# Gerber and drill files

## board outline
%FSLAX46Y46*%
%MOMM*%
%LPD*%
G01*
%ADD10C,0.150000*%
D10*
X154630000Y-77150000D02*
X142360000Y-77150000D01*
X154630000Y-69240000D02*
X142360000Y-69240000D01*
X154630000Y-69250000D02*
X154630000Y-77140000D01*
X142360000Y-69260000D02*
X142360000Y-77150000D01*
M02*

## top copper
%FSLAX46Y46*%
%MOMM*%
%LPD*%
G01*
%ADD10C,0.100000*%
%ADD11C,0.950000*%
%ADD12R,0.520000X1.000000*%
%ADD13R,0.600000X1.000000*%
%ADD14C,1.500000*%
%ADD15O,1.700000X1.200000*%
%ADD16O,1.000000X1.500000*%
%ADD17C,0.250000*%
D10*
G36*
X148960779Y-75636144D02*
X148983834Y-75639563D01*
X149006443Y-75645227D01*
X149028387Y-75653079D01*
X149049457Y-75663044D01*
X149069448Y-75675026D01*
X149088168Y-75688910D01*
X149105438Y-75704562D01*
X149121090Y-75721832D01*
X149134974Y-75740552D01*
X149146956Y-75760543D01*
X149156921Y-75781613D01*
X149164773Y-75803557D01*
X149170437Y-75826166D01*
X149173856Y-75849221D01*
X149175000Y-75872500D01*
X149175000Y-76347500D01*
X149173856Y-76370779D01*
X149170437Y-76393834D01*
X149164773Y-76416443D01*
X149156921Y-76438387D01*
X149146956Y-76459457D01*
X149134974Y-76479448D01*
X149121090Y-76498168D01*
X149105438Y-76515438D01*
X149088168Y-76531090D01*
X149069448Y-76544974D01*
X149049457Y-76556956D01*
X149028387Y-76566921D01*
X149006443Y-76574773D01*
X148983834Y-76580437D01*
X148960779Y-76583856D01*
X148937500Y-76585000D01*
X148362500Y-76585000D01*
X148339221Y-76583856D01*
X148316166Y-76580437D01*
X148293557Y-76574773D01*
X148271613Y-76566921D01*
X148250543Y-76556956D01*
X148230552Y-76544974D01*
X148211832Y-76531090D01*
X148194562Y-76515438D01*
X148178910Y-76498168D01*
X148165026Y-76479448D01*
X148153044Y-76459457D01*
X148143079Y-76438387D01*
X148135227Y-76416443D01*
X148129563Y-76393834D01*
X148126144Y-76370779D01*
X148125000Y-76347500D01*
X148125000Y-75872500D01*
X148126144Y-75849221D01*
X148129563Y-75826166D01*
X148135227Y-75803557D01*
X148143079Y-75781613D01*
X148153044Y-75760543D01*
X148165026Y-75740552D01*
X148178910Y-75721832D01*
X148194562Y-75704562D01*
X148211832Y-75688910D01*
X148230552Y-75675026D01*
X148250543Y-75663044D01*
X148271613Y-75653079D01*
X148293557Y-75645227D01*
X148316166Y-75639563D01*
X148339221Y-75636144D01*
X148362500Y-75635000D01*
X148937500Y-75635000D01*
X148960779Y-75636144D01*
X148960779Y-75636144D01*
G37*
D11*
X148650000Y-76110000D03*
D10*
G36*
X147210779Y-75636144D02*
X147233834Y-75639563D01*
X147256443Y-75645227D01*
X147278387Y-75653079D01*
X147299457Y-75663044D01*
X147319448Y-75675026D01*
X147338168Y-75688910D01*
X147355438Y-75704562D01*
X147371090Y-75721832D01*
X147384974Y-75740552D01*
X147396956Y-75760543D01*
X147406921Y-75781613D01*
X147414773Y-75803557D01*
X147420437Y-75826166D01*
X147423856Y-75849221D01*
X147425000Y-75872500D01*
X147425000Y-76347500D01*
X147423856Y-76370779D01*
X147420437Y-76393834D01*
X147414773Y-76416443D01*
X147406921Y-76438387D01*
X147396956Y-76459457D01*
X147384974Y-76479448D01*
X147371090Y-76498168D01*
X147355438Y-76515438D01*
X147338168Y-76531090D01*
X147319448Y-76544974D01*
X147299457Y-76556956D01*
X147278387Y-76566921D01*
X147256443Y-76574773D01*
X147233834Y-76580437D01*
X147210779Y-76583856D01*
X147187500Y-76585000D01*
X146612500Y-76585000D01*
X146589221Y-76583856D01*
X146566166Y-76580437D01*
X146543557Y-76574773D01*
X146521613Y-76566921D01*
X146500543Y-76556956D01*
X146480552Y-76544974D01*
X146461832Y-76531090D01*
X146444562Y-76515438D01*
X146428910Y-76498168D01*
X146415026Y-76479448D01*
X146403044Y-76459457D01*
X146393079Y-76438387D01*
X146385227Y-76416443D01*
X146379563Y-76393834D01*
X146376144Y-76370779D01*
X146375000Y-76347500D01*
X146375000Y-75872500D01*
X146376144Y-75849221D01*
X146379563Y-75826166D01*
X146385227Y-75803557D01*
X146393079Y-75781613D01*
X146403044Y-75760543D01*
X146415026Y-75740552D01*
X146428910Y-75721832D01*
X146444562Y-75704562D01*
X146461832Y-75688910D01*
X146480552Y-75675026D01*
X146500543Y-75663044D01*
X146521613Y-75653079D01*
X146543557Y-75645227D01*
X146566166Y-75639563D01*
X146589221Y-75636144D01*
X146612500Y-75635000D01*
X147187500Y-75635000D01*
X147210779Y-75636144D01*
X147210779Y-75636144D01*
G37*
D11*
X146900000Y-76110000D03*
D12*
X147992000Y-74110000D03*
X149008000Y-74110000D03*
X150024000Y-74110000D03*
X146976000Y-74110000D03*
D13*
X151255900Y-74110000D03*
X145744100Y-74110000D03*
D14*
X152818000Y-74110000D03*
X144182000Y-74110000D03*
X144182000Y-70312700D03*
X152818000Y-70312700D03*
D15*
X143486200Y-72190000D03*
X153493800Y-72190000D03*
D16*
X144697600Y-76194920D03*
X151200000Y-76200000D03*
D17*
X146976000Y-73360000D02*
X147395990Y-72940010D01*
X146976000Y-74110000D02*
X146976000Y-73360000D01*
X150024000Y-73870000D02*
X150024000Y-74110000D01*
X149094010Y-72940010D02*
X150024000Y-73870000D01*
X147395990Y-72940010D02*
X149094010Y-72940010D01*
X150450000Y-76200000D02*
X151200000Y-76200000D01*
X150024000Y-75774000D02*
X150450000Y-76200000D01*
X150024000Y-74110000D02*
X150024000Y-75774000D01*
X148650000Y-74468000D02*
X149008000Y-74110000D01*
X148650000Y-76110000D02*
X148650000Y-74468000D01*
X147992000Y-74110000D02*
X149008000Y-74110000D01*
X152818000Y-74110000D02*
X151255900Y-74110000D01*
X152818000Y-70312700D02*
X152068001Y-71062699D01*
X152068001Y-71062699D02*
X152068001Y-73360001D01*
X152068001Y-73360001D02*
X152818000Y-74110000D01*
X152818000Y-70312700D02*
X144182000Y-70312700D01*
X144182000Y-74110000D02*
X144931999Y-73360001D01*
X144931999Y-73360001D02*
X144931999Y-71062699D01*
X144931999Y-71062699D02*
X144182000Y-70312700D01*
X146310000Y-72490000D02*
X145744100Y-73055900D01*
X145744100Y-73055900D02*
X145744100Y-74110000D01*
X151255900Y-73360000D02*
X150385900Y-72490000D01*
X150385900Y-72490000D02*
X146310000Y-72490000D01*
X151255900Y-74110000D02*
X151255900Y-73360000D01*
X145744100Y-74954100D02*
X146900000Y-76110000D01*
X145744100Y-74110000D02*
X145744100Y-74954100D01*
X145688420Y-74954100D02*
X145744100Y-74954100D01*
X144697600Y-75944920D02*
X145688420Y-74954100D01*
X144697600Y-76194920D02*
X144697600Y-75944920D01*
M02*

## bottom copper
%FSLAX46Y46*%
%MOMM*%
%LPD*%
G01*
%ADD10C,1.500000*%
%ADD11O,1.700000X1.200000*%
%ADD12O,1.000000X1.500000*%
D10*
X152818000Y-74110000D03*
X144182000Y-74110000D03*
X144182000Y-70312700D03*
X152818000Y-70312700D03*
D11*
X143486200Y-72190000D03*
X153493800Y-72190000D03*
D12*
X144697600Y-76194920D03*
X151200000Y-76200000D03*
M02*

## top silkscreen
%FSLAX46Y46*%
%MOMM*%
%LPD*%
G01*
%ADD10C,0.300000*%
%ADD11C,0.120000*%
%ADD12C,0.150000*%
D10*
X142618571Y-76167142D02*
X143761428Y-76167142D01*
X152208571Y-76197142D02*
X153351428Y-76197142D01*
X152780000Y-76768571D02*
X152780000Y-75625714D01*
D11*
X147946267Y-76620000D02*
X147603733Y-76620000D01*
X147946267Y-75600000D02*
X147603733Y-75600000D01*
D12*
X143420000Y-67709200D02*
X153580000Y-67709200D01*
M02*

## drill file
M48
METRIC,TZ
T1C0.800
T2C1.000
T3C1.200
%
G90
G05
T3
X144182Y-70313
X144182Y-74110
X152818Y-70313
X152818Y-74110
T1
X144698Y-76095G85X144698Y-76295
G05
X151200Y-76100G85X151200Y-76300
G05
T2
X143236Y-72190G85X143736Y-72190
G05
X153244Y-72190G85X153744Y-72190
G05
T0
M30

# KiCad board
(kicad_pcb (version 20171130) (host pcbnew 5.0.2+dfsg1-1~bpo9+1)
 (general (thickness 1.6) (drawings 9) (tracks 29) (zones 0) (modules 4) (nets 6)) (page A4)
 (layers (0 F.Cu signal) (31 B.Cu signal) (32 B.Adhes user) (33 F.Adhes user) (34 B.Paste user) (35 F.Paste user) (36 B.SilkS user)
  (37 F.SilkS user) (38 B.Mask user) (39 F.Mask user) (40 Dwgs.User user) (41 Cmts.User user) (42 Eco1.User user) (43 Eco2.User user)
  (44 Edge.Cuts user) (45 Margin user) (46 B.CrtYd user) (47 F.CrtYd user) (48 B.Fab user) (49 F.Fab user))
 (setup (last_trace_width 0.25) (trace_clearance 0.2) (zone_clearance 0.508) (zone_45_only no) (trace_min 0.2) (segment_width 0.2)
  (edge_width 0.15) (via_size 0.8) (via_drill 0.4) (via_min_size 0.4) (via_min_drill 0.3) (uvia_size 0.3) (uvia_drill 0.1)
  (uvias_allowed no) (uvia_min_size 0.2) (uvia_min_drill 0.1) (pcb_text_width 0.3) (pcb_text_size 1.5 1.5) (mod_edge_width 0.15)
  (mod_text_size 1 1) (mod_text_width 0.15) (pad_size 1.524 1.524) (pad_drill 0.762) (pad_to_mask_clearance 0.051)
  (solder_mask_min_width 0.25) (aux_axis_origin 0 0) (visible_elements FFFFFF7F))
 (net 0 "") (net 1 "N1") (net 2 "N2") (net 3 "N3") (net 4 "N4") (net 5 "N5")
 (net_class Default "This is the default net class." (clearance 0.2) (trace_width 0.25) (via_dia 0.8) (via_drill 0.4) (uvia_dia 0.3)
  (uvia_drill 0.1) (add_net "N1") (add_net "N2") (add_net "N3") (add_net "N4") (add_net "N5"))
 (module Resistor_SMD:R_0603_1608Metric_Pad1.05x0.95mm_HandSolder (layer F.Cu) (at 147.775 76.11 180)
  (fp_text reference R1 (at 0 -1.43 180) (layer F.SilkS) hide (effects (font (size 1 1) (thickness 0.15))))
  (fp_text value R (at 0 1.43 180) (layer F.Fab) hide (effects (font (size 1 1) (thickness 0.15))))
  (fp_line (start -0.171267 -0.51) (end 0.171267 -0.51) (layer F.SilkS) (width 0.12))
  (fp_line (start -0.171267 0.51) (end 0.171267 0.51) (layer F.SilkS) (width 0.12))
  (pad 1 smd roundrect (at -0.875 0 180) (size 1.05 0.95) (layers F.Cu F.Paste F.Mask) (roundrect_rratio 0.25) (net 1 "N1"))
  (pad 2 smd roundrect (at 0.875 0 180) (size 1.05 0.95) (layers F.Cu F.Paste F.Mask) (roundrect_rratio 0.25) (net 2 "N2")))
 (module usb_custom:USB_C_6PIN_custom (layer F.Cu) (at 148.5 74.11)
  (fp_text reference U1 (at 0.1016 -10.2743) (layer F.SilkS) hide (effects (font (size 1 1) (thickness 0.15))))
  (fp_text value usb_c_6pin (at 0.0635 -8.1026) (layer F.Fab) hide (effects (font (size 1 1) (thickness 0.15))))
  (fp_line (start -5.08 -6.4008) (end 5.08 -6.4008) (layer F.SilkS) (width 0.15))
  (pad 3 smd rect (at -0.508 0) (size 0.52 1) (layers F.Cu F.Paste F.Mask) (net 1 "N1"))
  (pad 4 smd rect (at 0.508 0) (size 0.52 1) (layers F.Cu F.Paste F.Mask) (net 1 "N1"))
  (pad 2 smd rect (at 1.524 0) (size 0.52 1) (layers F.Cu F.Paste F.Mask) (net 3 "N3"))
  (pad 2 smd rect (at -1.524 0) (size 0.52 1) (layers F.Cu F.Paste F.Mask) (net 3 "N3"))
  (pad 1 smd rect (at 2.7559 0) (size 0.6 1) (layers F.Cu F.Paste F.Mask) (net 2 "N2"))
  (pad 1 smd rect (at -2.7559 0) (size 0.6 1) (layers F.Cu F.Paste F.Mask) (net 2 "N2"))
  (pad 1 thru_hole circle (at 4.318 0) (size 1.5 1.5) (drill 1.2) (layers *.Cu *.Mask) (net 2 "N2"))
  (pad 1 thru_hole circle (at -4.318 0) (size 1.5 1.5) (drill 1.2) (layers *.Cu *.Mask) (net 2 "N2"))
  (pad 1 thru_hole circle (at -4.318 -3.7973) (size 1.5 1.5) (drill 1.2) (layers *.Cu *.Mask) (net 2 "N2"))
  (pad 1 thru_hole circle (at 4.318 -3.7973) (size 1.5 1.5) (drill 1.2) (layers *.Cu *.Mask) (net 2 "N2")))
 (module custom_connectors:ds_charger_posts (layer F.Cu) (at 148.49 72.19)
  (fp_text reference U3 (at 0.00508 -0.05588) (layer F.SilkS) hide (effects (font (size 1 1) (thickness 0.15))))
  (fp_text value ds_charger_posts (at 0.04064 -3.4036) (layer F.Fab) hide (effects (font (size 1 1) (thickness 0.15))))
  (pad 1 thru_hole oval (at -5.0038 0) (size 1.7 1.2) (drill oval 1.5 1) (layers *.Cu *.Mask) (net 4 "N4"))
  (pad 2 thru_hole oval (at 5.0038 0) (size 1.7 1.2) (drill oval 1.5 1) (layers *.Cu *.Mask) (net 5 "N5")))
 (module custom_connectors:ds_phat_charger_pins (layer F.Cu) (at 147.44588 76.2)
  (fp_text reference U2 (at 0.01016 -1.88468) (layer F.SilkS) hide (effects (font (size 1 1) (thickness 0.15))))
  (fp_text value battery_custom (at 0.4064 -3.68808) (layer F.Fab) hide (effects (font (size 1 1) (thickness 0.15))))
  (pad 1 thru_hole oval (at -2.74828 -0.00508) (size 1 1.5) (drill oval 0.8 1) (layers *.Cu *.Mask) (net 2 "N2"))
  (pad 2 thru_hole oval (at 3.75412 0) (size 1 1.5) (drill oval 0.8 1) (layers *.Cu *.Mask) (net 3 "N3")))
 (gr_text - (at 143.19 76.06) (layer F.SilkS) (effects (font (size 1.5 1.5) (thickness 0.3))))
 (gr_line (start 154.63 77.15) (end 142.36 77.15) (layer Edge.Cuts) (width 0.15))
 (gr_line (start 154.63 69.24) (end 142.36 69.24) (layer Edge.Cuts) (width 0.15))
 (gr_line (start 154.63 69.25) (end 154.63 77.14) (layer Edge.Cuts) (width 0.15))
 (gr_line (start 142.36 69.26) (end 142.36 77.15) (layer Edge.Cuts) (width 0.15))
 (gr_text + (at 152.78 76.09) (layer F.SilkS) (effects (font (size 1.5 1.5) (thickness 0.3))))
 (segment (start 146.976 73.36) (end 147.39599 72.94001) (width 0.25) (layer F.Cu) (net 3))
 (segment (start 146.976 74.11) (end 146.976 73.36) (width 0.25) (layer F.Cu) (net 3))
 (segment (start 150.024 73.87) (end 150.024 74.11) (width 0.25) (layer F.Cu) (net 3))
 (segment (start 149.09401 72.94001) (end 150.024 73.87) (width 0.25) (layer F.Cu) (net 3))
 (segment (start 147.39599 72.94001) (end 149.09401 72.94001) (width 0.25) (layer F.Cu) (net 3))
 (segment (start 150.45 76.2) (end 151.2 76.2) (width 0.25) (layer F.Cu) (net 3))
 (segment (start 150.024 75.774) (end 150.45 76.2) (width 0.25) (layer F.Cu) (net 3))
 (segment (start 150.024 74.11) (end 150.024 75.774) (width 0.25) (layer F.Cu) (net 3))
 (segment (start 148.65 74.468) (end 149.008 74.11) (width 0.25) (layer F.Cu) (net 1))
 (segment (start 148.65 76.11) (end 148.65 74.468) (width 0.25) (layer F.Cu) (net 1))
 (segment (start 147.992 74.11) (end 149.008 74.11) (width 0.25) (layer F.Cu) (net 1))
 (segment (start 152.818 74.11) (end 151.2559 74.11) (width 0.25) (layer F.Cu) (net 2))
 (segment (start 152.818 70.3127) (end 152.068001 71.062699) (width 0.25) (layer F.Cu) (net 2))
 (segment (start 152.068001 71.062699) (end 152.068001 73.360001) (width 0.25) (layer F.Cu) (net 2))
 (segment (start 152.068001 73.360001) (end 152.818 74.11) (width 0.25) (layer F.Cu) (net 2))
 (segment (start 152.818 70.3127) (end 144.182 70.3127) (width 0.25) (layer F.Cu) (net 2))
 (segment (start 144.182 74.11) (end 144.931999 73.360001) (width 0.25) (layer F.Cu) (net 2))
 (segment (start 144.931999 73.360001) (end 144.931999 71.062699) (width 0.25) (layer F.Cu) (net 2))
 (segment (start 144.931999 71.062699) (end 144.182 70.3127) (width 0.25) (layer F.Cu) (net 2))
 (segment (start 146.31 72.49) (end 145.7441 73.0559) (width 0.25) (layer F.Cu) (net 2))
 (segment (start 145.7441 73.0559) (end 145.7441 74.11) (width 0.25) (layer F.Cu) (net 2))
 (segment (start 151.2559 73.36) (end 150.3859 72.49) (width 0.25) (layer F.Cu) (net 2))
 (segment (start 150.3859 72.49) (end 146.31 72.49) (width 0.25) (layer F.Cu) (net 2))
 (segment (start 151.2559 74.11) (end 151.2559 73.36) (width 0.25) (layer F.Cu) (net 2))
 (segment (start 145.7441 74.9541) (end 146.9 76.11) (width 0.25) (layer F.Cu) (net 2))
 (segment (start 145.7441 74.11) (end 145.7441 74.9541) (width 0.25) (layer F.Cu) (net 2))
 (segment (start 145.68842 74.9541) (end 145.7441 74.9541) (width 0.25) (layer F.Cu) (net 2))
 (segment (start 144.6976 75.94492) (end 145.68842 74.9541) (width 0.25) (layer F.Cu) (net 2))
 (segment (start 144.6976 76.19492) (end 144.6976 75.94492) (width 0.25) (layer F.Cu) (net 2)))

